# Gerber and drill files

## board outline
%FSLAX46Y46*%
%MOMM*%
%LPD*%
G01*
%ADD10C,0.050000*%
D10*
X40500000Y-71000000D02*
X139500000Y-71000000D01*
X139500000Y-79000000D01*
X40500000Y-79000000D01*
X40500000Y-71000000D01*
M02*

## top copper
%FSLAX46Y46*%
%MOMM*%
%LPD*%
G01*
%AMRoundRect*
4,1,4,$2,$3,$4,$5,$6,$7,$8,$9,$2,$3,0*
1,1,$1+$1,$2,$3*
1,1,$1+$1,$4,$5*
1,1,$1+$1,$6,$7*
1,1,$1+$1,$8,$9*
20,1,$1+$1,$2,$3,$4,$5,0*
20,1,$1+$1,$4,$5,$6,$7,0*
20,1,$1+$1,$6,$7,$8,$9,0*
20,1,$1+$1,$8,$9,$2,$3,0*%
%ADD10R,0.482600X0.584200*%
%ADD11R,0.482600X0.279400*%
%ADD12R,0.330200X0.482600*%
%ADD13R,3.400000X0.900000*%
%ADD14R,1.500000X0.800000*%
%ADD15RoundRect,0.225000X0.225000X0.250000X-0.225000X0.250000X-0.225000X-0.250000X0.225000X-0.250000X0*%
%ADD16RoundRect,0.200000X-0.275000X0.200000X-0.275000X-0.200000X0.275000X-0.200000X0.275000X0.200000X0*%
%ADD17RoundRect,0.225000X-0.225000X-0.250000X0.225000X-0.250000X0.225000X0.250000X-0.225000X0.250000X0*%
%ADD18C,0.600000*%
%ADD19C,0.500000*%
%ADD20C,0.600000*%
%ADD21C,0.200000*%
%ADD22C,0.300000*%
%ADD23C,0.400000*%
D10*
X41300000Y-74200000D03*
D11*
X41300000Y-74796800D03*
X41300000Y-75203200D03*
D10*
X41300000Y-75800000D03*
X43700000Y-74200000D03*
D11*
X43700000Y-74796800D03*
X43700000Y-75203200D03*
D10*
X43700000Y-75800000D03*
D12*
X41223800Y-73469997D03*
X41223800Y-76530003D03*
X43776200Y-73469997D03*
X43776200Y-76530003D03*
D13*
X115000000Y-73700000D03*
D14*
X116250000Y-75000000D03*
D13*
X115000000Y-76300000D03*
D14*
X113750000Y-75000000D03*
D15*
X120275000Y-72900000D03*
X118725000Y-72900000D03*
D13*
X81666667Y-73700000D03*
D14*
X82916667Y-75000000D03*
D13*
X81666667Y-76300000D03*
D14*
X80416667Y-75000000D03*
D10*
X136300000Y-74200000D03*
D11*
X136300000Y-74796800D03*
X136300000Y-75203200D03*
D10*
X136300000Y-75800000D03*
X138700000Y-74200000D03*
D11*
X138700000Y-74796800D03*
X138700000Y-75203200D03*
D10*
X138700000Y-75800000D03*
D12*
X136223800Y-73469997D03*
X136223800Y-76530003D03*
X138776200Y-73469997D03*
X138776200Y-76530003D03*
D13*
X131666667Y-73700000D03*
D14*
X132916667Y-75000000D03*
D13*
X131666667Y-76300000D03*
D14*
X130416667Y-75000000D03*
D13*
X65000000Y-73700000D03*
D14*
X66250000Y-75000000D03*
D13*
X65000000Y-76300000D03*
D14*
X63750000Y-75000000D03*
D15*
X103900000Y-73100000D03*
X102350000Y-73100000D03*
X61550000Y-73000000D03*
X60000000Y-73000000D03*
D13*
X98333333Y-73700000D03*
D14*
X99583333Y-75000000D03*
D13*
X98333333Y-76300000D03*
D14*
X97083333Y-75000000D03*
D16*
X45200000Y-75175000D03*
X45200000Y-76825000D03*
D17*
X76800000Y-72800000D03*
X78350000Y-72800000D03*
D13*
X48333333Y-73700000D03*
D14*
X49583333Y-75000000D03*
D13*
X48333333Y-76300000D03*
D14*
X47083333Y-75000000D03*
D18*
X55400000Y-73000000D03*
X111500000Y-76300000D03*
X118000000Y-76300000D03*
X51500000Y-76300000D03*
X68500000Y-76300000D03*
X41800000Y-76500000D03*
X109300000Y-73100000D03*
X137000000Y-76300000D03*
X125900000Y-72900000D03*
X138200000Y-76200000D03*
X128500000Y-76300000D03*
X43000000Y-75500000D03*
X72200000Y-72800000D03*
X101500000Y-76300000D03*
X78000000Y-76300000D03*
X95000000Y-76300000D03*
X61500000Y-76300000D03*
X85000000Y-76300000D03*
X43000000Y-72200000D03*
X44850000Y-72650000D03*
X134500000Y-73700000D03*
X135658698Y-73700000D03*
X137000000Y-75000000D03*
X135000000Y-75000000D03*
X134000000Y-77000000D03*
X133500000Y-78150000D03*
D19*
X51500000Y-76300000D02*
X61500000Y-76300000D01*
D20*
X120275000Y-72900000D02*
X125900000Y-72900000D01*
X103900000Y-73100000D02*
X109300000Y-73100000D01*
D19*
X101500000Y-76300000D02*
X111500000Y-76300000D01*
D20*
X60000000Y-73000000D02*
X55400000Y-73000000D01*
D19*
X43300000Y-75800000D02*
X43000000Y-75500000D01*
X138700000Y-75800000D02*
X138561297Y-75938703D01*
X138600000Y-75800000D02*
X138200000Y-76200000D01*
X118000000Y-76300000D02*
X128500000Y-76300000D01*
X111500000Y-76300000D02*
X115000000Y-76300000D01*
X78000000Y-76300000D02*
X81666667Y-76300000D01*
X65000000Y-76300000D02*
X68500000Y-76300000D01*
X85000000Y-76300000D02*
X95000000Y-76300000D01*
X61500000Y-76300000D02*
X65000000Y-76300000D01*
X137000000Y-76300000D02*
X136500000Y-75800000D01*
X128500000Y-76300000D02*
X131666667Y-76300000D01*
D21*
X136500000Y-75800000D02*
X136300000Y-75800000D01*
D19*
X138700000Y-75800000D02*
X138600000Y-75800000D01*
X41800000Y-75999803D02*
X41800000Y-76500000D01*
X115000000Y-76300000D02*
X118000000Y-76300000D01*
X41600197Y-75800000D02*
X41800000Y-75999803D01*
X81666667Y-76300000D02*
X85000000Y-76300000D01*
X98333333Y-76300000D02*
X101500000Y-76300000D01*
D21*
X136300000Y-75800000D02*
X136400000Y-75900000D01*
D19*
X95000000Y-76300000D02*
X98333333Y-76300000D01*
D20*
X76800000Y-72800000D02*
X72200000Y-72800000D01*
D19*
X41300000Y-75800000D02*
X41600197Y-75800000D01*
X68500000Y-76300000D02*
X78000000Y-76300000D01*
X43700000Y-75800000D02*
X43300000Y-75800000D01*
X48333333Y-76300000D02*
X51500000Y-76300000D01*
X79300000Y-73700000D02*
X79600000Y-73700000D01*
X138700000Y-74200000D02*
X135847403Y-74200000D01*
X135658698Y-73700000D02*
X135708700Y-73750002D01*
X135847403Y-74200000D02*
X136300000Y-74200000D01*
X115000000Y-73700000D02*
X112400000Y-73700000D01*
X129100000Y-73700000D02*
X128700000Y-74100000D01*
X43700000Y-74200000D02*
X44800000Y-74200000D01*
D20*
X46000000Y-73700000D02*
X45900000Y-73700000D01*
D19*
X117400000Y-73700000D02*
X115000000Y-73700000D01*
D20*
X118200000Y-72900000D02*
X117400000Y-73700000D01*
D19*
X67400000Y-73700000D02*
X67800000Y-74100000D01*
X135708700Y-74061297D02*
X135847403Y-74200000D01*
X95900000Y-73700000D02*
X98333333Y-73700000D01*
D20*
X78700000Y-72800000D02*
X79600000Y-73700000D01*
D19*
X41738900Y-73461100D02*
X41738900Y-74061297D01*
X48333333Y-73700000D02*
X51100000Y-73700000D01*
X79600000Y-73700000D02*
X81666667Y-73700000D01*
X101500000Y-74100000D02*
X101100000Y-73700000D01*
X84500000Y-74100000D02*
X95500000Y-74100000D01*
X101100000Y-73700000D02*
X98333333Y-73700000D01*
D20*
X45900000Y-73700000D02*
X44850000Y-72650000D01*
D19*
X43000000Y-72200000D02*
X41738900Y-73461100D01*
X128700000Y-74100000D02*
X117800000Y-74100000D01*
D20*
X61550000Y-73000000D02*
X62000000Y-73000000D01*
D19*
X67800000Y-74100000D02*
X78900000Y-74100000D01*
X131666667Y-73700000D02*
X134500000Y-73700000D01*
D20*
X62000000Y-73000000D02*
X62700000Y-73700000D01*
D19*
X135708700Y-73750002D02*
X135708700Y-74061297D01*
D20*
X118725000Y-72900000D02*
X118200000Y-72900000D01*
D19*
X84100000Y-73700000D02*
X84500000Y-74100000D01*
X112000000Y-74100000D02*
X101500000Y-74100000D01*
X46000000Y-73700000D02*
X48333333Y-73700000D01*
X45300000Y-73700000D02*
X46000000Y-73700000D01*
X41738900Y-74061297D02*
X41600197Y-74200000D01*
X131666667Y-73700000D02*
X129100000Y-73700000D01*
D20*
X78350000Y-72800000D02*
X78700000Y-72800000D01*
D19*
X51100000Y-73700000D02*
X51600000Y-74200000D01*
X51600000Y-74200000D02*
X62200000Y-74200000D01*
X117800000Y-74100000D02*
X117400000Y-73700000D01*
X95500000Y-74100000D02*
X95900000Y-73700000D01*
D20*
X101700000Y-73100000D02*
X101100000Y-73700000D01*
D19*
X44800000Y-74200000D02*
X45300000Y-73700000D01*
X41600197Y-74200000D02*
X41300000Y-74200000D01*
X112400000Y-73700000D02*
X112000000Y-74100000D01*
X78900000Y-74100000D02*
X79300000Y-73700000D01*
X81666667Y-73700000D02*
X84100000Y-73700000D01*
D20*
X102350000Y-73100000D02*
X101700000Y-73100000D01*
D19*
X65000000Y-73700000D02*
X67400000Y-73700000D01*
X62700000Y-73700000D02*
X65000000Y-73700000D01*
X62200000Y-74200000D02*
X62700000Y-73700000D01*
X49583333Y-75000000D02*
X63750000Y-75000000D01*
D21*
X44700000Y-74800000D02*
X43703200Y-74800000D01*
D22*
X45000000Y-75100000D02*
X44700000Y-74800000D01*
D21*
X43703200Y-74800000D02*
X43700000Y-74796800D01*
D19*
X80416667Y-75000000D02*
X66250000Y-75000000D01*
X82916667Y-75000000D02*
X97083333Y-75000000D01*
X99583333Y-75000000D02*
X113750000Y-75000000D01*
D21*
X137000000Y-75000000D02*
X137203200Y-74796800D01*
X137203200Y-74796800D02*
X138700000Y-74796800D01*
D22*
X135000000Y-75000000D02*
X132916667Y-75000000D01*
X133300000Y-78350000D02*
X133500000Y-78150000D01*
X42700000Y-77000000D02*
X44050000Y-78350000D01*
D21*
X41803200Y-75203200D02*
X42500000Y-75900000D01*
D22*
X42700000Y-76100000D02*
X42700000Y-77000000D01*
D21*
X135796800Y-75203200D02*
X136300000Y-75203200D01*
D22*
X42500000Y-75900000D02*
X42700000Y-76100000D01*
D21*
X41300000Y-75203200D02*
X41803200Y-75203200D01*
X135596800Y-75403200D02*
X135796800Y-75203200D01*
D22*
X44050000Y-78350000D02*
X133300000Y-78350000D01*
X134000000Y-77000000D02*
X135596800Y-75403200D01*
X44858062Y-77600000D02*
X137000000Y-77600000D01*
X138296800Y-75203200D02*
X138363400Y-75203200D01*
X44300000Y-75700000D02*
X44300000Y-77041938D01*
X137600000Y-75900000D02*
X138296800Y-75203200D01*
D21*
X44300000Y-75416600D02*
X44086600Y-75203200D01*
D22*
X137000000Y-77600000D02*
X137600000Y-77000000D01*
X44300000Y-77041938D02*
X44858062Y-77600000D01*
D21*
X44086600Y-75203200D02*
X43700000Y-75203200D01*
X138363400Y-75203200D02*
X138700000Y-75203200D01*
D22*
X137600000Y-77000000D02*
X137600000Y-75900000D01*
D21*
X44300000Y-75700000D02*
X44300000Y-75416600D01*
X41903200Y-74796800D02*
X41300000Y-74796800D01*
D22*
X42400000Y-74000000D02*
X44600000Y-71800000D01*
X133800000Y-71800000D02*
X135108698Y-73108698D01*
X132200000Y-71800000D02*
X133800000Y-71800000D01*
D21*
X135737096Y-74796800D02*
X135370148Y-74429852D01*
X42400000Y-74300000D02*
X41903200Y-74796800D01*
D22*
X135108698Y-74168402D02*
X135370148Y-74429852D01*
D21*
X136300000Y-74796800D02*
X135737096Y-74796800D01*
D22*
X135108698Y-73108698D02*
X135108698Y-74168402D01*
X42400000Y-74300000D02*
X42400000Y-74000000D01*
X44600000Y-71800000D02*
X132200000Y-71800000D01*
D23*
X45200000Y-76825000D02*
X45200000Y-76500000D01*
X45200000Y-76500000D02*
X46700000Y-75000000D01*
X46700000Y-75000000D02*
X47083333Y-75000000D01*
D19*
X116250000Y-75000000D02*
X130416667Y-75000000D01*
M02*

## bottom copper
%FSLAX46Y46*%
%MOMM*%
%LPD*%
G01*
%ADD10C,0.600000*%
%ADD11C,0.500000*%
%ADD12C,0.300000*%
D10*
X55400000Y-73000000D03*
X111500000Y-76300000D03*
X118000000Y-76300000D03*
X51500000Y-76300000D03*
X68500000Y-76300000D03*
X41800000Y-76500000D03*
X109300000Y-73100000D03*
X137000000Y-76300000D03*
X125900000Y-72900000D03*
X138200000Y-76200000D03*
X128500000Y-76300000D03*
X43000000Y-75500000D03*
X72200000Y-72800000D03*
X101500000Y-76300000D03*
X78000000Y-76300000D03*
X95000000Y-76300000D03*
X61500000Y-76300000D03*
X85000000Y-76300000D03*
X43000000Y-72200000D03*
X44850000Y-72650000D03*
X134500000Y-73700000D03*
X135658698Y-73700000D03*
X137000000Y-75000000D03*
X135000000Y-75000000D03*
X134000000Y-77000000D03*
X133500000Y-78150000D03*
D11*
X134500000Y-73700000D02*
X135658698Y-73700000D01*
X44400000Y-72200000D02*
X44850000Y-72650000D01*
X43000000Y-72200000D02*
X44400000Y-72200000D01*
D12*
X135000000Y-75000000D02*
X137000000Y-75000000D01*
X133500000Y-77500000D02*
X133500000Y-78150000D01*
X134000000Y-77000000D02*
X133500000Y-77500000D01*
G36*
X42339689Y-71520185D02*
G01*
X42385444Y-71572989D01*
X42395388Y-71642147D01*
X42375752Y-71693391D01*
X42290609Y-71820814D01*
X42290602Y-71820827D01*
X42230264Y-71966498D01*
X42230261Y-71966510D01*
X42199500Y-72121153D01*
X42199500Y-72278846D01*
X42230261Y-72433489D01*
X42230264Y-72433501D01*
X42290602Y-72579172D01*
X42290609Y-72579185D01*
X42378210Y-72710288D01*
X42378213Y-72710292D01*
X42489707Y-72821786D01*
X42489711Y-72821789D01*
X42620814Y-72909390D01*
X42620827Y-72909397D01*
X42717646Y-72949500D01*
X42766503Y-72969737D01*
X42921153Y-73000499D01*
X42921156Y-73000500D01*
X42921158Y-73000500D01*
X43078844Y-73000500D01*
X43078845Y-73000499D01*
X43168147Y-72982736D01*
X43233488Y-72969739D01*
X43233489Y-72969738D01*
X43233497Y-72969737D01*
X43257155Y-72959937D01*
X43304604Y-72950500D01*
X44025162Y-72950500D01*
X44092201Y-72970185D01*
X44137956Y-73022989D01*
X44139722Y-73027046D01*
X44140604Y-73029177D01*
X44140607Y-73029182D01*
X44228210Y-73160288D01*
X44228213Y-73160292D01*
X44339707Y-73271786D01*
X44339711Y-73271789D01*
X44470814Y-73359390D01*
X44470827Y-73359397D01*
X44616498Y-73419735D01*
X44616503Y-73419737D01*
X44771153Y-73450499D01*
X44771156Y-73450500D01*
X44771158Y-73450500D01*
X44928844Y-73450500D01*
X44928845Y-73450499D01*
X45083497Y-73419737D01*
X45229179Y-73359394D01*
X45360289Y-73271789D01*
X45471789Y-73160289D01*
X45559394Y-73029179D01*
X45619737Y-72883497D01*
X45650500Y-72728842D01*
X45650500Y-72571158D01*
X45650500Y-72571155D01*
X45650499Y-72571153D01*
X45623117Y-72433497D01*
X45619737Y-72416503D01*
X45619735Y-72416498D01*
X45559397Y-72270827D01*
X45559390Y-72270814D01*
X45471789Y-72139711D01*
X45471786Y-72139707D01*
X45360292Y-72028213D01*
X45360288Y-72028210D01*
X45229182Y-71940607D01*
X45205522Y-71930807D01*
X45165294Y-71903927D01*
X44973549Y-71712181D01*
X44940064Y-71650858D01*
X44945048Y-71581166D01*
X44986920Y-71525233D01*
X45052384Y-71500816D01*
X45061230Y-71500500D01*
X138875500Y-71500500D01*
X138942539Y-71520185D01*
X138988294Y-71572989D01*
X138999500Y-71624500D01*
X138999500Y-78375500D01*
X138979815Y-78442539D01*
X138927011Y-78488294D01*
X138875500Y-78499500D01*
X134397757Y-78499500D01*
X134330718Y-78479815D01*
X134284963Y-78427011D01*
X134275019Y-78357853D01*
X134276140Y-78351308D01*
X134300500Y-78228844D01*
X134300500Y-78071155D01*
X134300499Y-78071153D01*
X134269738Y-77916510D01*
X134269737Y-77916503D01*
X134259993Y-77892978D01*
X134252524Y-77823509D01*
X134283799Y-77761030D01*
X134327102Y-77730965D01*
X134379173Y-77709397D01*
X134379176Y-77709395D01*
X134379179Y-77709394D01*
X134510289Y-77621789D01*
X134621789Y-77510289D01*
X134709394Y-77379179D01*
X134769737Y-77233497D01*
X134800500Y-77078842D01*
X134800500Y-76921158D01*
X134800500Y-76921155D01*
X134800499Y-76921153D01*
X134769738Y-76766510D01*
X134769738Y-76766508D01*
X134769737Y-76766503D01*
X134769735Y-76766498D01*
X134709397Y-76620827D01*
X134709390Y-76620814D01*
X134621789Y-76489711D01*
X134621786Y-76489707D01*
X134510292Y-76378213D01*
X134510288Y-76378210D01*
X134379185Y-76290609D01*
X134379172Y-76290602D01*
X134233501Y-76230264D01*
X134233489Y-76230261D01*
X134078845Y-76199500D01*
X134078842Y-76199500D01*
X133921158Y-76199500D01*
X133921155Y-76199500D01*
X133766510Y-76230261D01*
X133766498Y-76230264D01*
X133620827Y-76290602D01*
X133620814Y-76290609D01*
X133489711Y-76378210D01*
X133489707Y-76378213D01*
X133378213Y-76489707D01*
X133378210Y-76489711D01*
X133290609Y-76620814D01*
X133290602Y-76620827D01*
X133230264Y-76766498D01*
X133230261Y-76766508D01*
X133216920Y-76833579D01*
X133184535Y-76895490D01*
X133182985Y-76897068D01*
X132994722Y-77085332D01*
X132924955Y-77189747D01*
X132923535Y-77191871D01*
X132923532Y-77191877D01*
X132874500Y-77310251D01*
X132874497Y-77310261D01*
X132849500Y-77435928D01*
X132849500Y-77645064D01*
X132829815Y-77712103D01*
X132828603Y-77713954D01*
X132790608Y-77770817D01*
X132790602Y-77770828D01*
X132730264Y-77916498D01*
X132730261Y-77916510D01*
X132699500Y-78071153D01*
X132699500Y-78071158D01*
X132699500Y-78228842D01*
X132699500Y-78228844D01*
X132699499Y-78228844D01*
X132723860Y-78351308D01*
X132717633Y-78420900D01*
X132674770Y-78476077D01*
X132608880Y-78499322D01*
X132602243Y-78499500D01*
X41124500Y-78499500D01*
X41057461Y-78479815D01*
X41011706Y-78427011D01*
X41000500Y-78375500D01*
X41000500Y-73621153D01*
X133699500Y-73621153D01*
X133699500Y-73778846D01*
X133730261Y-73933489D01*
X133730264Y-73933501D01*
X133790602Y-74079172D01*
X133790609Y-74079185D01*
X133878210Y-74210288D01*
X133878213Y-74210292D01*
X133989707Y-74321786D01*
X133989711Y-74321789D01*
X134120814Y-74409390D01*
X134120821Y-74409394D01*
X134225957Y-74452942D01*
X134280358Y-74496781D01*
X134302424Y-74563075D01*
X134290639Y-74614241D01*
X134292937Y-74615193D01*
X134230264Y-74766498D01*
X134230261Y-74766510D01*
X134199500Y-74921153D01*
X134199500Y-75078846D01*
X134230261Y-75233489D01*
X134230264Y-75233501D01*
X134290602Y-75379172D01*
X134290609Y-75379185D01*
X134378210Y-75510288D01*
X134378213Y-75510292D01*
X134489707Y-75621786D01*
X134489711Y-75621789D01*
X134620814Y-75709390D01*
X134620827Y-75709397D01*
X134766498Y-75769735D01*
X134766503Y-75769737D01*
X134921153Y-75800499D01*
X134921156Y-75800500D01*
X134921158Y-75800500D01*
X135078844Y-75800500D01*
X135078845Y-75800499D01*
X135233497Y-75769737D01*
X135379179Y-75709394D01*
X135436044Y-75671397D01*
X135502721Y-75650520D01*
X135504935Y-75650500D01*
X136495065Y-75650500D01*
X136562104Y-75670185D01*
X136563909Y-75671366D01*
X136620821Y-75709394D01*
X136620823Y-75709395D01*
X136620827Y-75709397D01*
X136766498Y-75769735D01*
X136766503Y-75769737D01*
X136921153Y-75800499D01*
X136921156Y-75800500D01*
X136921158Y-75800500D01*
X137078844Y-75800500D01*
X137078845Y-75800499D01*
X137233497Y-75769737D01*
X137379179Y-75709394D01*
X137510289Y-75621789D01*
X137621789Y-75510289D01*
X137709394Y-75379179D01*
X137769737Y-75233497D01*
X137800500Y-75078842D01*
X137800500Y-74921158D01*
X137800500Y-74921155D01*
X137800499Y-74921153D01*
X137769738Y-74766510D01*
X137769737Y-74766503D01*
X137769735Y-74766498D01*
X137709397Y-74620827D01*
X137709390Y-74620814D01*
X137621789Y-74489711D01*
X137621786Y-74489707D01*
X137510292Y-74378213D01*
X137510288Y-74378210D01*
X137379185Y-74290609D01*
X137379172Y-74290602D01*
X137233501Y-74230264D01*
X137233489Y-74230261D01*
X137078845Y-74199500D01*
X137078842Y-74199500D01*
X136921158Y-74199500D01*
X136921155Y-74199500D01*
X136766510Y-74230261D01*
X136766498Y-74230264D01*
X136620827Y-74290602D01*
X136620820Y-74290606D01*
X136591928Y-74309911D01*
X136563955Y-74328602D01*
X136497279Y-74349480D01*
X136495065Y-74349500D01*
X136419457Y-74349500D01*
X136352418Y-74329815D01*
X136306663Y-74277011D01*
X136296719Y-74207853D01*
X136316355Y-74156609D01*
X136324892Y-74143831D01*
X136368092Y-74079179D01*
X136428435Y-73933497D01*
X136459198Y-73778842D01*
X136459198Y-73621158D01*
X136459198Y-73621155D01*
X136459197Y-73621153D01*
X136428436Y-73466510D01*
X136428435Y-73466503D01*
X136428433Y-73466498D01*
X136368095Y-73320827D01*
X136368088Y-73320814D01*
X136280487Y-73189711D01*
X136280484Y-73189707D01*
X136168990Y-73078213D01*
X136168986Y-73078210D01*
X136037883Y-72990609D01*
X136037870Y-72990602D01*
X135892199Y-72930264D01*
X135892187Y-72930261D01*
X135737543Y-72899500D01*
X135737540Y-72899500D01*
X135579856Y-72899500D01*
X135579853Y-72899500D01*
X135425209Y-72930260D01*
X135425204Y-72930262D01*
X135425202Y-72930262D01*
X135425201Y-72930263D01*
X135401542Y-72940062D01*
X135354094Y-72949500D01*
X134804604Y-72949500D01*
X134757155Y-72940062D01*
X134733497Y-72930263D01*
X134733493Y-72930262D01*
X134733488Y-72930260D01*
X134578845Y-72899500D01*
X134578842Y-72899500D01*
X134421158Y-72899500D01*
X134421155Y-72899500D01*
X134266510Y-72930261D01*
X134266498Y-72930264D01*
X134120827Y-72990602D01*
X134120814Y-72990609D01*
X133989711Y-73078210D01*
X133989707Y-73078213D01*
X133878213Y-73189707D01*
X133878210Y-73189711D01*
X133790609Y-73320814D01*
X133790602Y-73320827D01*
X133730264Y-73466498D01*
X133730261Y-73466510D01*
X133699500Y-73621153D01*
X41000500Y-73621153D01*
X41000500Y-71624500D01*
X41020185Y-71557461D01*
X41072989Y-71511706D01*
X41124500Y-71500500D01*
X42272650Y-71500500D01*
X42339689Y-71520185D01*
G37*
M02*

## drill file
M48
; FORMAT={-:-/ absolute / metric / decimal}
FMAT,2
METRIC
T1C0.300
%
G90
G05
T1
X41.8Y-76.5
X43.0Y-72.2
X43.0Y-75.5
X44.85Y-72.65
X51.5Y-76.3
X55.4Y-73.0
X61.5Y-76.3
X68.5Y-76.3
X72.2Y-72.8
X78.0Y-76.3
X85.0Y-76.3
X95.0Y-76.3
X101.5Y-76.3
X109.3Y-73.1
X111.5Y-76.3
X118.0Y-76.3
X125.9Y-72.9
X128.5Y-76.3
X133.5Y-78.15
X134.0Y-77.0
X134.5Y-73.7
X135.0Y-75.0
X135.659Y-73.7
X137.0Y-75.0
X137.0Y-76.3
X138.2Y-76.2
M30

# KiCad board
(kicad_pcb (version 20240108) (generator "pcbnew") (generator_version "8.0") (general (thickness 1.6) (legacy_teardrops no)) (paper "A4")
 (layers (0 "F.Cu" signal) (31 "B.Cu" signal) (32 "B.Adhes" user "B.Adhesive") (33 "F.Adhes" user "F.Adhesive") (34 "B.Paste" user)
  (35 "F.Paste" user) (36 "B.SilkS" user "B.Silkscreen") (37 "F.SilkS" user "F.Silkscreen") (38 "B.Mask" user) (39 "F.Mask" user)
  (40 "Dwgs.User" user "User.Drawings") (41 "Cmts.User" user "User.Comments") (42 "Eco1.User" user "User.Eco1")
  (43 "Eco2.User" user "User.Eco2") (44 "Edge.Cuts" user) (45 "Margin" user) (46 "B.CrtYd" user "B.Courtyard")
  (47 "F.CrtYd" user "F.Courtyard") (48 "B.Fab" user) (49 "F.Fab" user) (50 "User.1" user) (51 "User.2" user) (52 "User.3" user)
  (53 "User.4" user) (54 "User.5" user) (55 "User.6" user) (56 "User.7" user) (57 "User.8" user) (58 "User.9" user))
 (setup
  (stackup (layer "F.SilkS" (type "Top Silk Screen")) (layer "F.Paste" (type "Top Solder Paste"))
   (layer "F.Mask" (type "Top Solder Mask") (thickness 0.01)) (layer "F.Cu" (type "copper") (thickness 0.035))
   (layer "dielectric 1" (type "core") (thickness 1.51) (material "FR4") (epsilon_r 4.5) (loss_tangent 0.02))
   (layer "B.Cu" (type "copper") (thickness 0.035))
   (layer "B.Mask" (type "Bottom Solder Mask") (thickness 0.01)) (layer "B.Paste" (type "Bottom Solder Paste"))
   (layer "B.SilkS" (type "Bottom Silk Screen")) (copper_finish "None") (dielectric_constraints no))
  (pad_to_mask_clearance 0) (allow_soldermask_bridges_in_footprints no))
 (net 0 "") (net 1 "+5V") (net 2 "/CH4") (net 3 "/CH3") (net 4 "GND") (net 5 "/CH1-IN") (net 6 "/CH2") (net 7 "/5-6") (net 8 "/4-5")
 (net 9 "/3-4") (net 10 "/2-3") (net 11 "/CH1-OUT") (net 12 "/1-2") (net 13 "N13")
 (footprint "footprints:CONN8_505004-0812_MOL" (layer "F.Cu") (at 42.5 75 90)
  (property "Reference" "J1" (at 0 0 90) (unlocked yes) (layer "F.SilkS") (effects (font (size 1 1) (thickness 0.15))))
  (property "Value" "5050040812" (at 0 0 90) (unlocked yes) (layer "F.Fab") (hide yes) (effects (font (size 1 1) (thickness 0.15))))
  (pad "1" smd rect (at 0.8 -1.2 90) (size 0.5842 0.4826) (layers "F.Cu" "F.Paste" "F.Mask") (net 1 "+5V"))
  (pad "2" smd rect (at 0.2032 -1.2 90) (size 0.2794 0.4826) (layers "F.Cu" "F.Paste" "F.Mask") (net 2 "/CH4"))
  (pad "3" smd rect (at -0.2032 -1.2 90) (size 0.2794 0.4826) (layers "F.Cu" "F.Paste" "F.Mask") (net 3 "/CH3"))
  (pad "4" smd rect (at -0.8 -1.2 90) (size 0.5842 0.4826) (layers "F.Cu" "F.Paste" "F.Mask") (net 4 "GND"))
  (pad "5" smd rect (at 0.8 1.2 90) (size 0.5842 0.4826) (layers "F.Cu" "F.Paste" "F.Mask") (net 1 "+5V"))
  (pad "6" smd rect (at 0.2032 1.2 90) (size 0.2794 0.4826) (layers "F.Cu" "F.Paste" "F.Mask") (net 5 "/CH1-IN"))
  (pad "7" smd rect (at -0.2032 1.2 90) (size 0.2794 0.4826) (layers "F.Cu" "F.Paste" "F.Mask") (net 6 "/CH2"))
  (pad "8" smd rect (at -0.8 1.2 90) (size 0.5842 0.4826) (layers "F.Cu" "F.Paste" "F.Mask") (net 4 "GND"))
  (pad "9" smd rect (at 1.530003 -1.2762 90) (size 0.4826 0.3302) (layers "F.Cu" "F.Paste" "F.Mask"))
  (pad "10" smd rect (at -1.530003 -1.2762 90) (size 0.4826 0.3302) (layers "F.Cu" "F.Paste" "F.Mask"))
  (pad "11" smd rect (at 1.530003 1.2762 90) (size 0.4826 0.3302) (layers "F.Cu" "F.Paste" "F.Mask"))
  (pad "12" smd rect (at -1.530003 1.2762 90) (size 0.4826 0.3302) (layers "F.Cu" "F.Paste" "F.Mask")))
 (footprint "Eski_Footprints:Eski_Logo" (layer "F.Cu") (at 90 76.9)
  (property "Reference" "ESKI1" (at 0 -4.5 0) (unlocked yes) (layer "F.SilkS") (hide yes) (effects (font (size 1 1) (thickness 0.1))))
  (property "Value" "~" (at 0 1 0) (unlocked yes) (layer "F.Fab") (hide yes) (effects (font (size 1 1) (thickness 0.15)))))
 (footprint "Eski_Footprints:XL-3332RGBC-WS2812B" (layer "F.Cu") (at 115 75)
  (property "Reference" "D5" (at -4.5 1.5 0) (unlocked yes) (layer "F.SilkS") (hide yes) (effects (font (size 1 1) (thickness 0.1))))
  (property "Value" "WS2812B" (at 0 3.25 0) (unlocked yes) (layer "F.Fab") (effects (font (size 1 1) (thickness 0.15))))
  (pad "1" smd rect (at 0 -1.3) (size 3.4 0.9) (layers "F.Cu" "F.Paste" "F.Mask") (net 1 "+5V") (thermal_bridge_angle 45))
  (pad "2" smd rect (at 1.25 0) (size 1.5 0.8) (layers "F.Cu" "F.Paste" "F.Mask") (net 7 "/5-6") (thermal_bridge_angle 45))
  (pad "3" smd rect (at 0 1.3) (size 3.4 0.9) (layers "F.Cu" "F.Paste" "F.Mask") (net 4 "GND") (thermal_bridge_angle 45))
  (pad "4" smd rect (at -1.25 0) (size 1.5 0.8) (layers "F.Cu" "F.Paste" "F.Mask") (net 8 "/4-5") (thermal_bridge_angle 45)))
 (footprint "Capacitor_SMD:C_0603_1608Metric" (layer "F.Cu") (at 119.5 72.9 180)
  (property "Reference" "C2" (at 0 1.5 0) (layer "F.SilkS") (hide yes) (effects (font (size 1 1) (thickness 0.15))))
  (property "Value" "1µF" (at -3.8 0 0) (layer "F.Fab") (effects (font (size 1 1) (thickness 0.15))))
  (pad "1" smd roundrect (at -0.775 0 180) (size 0.9 0.95) (layers "F.Cu" "F.Paste" "F.Mask") (roundrect_rratio 0.25) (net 4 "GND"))
  (pad "2" smd roundrect (at 0.775 0 180) (size 0.9 0.95) (layers "F.Cu" "F.Paste" "F.Mask") (roundrect_rratio 0.25) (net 1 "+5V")))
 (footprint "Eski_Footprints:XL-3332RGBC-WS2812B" (layer "F.Cu") (at 81.666667 75)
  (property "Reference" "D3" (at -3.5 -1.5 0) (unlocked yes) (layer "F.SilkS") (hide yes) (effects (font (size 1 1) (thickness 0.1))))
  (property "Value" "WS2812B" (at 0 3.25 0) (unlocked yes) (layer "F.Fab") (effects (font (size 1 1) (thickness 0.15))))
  (pad "1" smd rect (at 0 -1.3) (size 3.4 0.9) (layers "F.Cu" "F.Paste" "F.Mask") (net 1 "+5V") (thermal_bridge_angle 45))
  (pad "2" smd rect (at 1.25 0) (size 1.5 0.8) (layers "F.Cu" "F.Paste" "F.Mask") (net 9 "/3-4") (thermal_bridge_angle 45))
  (pad "3" smd rect (at 0 1.3) (size 3.4 0.9) (layers "F.Cu" "F.Paste" "F.Mask") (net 4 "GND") (thermal_bridge_angle 45))
  (pad "4" smd rect (at -1.25 0) (size 1.5 0.8) (layers "F.Cu" "F.Paste" "F.Mask") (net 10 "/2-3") (thermal_bridge_angle 45)))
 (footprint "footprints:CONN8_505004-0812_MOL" (layer "F.Cu") (at 137.5 75 90)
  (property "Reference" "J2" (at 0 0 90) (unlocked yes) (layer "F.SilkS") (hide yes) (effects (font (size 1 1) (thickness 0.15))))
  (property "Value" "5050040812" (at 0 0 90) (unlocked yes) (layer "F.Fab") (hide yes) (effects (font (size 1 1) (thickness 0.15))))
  (pad "1" smd rect (at 0.8 -1.2 90) (size 0.5842 0.4826) (layers "F.Cu" "F.Paste" "F.Mask") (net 1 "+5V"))
  (pad "2" smd rect (at 0.2032 -1.2 90) (size 0.2794 0.4826) (layers "F.Cu" "F.Paste" "F.Mask") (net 2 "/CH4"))
  (pad "3" smd rect (at -0.2032 -1.2 90) (size 0.2794 0.4826) (layers "F.Cu" "F.Paste" "F.Mask") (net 3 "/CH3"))
  (pad "4" smd rect (at -0.8 -1.2 90) (size 0.5842 0.4826) (layers "F.Cu" "F.Paste" "F.Mask") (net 4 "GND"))
  (pad "5" smd rect (at 0.8 1.2 90) (size 0.5842 0.4826) (layers "F.Cu" "F.Paste" "F.Mask") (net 1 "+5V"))
  (pad "6" smd rect (at 0.2032 1.2 90) (size 0.2794 0.4826) (layers "F.Cu" "F.Paste" "F.Mask") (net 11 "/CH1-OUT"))
  (pad "7" smd rect (at -0.2032 1.2 90) (size 0.2794 0.4826) (layers "F.Cu" "F.Paste" "F.Mask") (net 6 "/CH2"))
  (pad "8" smd rect (at -0.8 1.2 90) (size 0.5842 0.4826) (layers "F.Cu" "F.Paste" "F.Mask") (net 4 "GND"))
  (pad "9" smd rect (at 1.530003 -1.2762 90) (size 0.4826 0.3302) (layers "F.Cu" "F.Paste" "F.Mask"))
  (pad "10" smd rect (at -1.530003 -1.2762 90) (size 0.4826 0.3302) (layers "F.Cu" "F.Paste" "F.Mask"))
  (pad "11" smd rect (at 1.530003 1.2762 90) (size 0.4826 0.3302) (layers "F.Cu" "F.Paste" "F.Mask"))
  (pad "12" smd rect (at -1.530003 1.2762 90) (size 0.4826 0.3302) (layers "F.Cu" "F.Paste" "F.Mask")))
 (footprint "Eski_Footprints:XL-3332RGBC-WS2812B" (layer "F.Cu") (at 131.666667 75)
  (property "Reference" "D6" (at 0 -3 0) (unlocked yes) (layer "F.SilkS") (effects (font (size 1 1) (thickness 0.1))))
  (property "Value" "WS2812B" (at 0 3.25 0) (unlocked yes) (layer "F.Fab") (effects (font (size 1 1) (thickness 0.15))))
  (pad "1" smd rect (at 0 -1.3) (size 3.4 0.9) (layers "F.Cu" "F.Paste" "F.Mask") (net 1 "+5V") (thermal_bridge_angle 45))
  (pad "2" smd rect (at 1.25 0) (size 1.5 0.8) (layers "F.Cu" "F.Paste" "F.Mask") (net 11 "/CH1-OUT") (thermal_bridge_angle 45))
  (pad "3" smd rect (at 0 1.3) (size 3.4 0.9) (layers "F.Cu" "F.Paste" "F.Mask") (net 4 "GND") (thermal_bridge_angle 45))
  (pad "4" smd rect (at -1.25 0) (size 1.5 0.8) (layers "F.Cu" "F.Paste" "F.Mask") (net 7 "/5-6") (thermal_bridge_angle 45)))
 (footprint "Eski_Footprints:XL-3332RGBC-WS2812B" (layer "F.Cu") (at 65 75)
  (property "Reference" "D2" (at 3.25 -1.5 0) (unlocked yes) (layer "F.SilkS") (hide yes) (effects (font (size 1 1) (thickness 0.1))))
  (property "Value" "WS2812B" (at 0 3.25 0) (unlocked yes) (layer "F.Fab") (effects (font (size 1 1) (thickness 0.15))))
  (pad "1" smd rect (at 0 -1.3) (size 3.4 0.9) (layers "F.Cu" "F.Paste" "F.Mask") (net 1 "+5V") (thermal_bridge_angle 45))
  (pad "2" smd rect (at 1.25 0) (size 1.5 0.8) (layers "F.Cu" "F.Paste" "F.Mask") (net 10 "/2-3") (thermal_bridge_angle 45))
  (pad "3" smd rect (at 0 1.3) (size 3.4 0.9) (layers "F.Cu" "F.Paste" "F.Mask") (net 4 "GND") (thermal_bridge_angle 45))
  (pad "4" smd rect (at -1.25 0) (size 1.5 0.8) (layers "F.Cu" "F.Paste" "F.Mask") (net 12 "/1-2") (thermal_bridge_angle 45)))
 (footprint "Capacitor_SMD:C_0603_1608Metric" (layer "F.Cu") (at 103.125 73.1 180)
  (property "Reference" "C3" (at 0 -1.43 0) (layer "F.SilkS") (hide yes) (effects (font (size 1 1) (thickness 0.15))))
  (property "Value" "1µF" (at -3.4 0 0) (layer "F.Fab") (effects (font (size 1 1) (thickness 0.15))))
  (pad "1" smd roundrect (at -0.775 0 180) (size 0.9 0.95) (layers "F.Cu" "F.Paste" "F.Mask") (roundrect_rratio 0.25) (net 4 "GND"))
  (pad "2" smd roundrect (at 0.775 0 180) (size 0.9 0.95) (layers "F.Cu" "F.Paste" "F.Mask") (roundrect_rratio 0.25) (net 1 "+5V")))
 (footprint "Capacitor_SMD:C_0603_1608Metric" (layer "F.Cu") (at 60.775 73 180)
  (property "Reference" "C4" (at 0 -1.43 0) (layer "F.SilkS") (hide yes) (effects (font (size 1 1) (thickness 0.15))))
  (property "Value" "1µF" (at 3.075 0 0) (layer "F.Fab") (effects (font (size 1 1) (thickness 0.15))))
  (pad "1" smd roundrect (at -0.775 0 180) (size 0.9 0.95) (layers "F.Cu" "F.Paste" "F.Mask") (roundrect_rratio 0.25) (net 1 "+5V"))
  (pad "2" smd roundrect (at 0.775 0 180) (size 0.9 0.95) (layers "F.Cu" "F.Paste" "F.Mask") (roundrect_rratio 0.25) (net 4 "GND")))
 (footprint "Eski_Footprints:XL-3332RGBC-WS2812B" (layer "F.Cu") (at 98.333333 75)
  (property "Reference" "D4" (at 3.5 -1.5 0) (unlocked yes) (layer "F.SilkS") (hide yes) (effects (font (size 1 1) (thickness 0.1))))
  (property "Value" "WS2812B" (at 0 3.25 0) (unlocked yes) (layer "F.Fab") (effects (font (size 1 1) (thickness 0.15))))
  (pad "1" smd rect (at 0 -1.3) (size 3.4 0.9) (layers "F.Cu" "F.Paste" "F.Mask") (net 1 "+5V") (thermal_bridge_angle 45))
  (pad "2" smd rect (at 1.25 0) (size 1.5 0.8) (layers "F.Cu" "F.Paste" "F.Mask") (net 8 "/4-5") (thermal_bridge_angle 45))
  (pad "3" smd rect (at 0 1.3) (size 3.4 0.9) (layers "F.Cu" "F.Paste" "F.Mask") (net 4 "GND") (thermal_bridge_angle 45))
  (pad "4" smd rect (at -1.25 0) (size 1.5 0.8) (layers "F.Cu" "F.Paste" "F.Mask") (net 9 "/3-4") (thermal_bridge_angle 45)))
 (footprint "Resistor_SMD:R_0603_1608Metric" (layer "F.Cu") (at 45.2 76 -90)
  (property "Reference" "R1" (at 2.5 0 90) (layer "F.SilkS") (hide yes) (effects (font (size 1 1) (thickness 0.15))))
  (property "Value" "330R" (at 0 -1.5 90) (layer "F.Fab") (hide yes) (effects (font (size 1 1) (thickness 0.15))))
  (pad "1" smd roundrect (at -0.825 0 270) (size 0.8 0.95) (layers "F.Cu" "F.Paste" "F.Mask") (roundrect_rratio 0.25) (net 5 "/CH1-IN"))
  (pad "2" smd roundrect (at 0.825 0 270) (size 0.8 0.95) (layers "F.Cu" "F.Paste" "F.Mask") (roundrect_rratio 0.25) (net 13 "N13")))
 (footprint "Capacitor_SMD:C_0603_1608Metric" (layer "F.Cu") (at 77.575 72.8)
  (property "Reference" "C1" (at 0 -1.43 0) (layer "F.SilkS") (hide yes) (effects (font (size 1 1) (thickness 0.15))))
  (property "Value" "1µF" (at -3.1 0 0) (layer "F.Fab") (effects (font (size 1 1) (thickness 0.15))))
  (pad "1" smd roundrect (at -0.775 0) (size 0.9 0.95) (layers "F.Cu" "F.Paste" "F.Mask") (roundrect_rratio 0.25) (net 4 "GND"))
  (pad "2" smd roundrect (at 0.775 0) (size 0.9 0.95) (layers "F.Cu" "F.Paste" "F.Mask") (roundrect_rratio 0.25) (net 1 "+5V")))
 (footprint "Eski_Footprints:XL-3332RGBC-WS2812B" (layer "F.Cu") (at 48.333333 75)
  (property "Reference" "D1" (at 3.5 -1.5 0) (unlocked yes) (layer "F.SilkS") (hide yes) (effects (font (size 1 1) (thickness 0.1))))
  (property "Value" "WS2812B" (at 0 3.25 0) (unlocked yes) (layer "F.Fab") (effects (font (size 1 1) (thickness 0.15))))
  (pad "1" smd rect (at 0 -1.3) (size 3.4 0.9) (layers "F.Cu" "F.Paste" "F.Mask") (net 1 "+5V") (thermal_bridge_angle 45))
  (pad "2" smd rect (at 1.25 0) (size 1.5 0.8) (layers "F.Cu" "F.Paste" "F.Mask") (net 12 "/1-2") (thermal_bridge_angle 45))
  (pad "3" smd rect (at 0 1.3) (size 3.4 0.9) (layers "F.Cu" "F.Paste" "F.Mask") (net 4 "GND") (thermal_bridge_angle 45))
  (pad "4" smd rect (at -1.25 0) (size 1.5 0.8) (layers "F.Cu" "F.Paste" "F.Mask") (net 13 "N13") (thermal_bridge_angle 45)))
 (gr_rect (start 40.5 71) (end 139.5 79) (stroke (width 0.05) (type default)) (fill none) (layer "Edge.Cuts"))
 (segment (start 51.5 76.3) (end 61.5 76.3) (width 0.5) (layer "F.Cu") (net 4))
 (segment (start 120.275 72.9) (end 125.9 72.9) (width 0.6) (layer "F.Cu") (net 4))
 (segment (start 103.9 73.1) (end 109.3 73.1) (width 0.6) (layer "F.Cu") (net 4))
 (segment (start 101.5 76.3) (end 111.5 76.3) (width 0.5) (layer "F.Cu") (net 4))
 (segment (start 60 73) (end 55.4 73) (width 0.6) (layer "F.Cu") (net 4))
 (segment (start 43.3 75.8) (end 43 75.5) (width 0.5) (layer "F.Cu") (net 4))
 (segment (start 138.7 75.8) (end 138.561297 75.938703) (width 0.5) (layer "F.Cu") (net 4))
 (segment (start 138.6 75.8) (end 138.2 76.2) (width 0.5) (layer "F.Cu") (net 4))
 (segment (start 118 76.3) (end 128.5 76.3) (width 0.5) (layer "F.Cu") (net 4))
 (segment (start 111.5 76.3) (end 115 76.3) (width 0.5) (layer "F.Cu") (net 4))
 (segment (start 78 76.3) (end 81.666667 76.3) (width 0.5) (layer "F.Cu") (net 4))
 (segment (start 65 76.3) (end 68.5 76.3) (width 0.5) (layer "F.Cu") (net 4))
 (segment (start 85 76.3) (end 95 76.3) (width 0.5) (layer "F.Cu") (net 4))
 (segment (start 61.5 76.3) (end 65 76.3) (width 0.5) (layer "F.Cu") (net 4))
 (segment (start 137 76.3) (end 136.5 75.8) (width 0.5) (layer "F.Cu") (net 4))
 (segment (start 128.5 76.3) (end 131.666667 76.3) (width 0.5) (layer "F.Cu") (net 4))
 (segment (start 136.5 75.8) (end 136.3 75.8) (width 0.2) (layer "F.Cu") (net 4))
 (segment (start 138.7 75.8) (end 138.6 75.8) (width 0.5) (layer "F.Cu") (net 4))
 (segment (start 41.8 75.999803) (end 41.8 76.5) (width 0.5) (layer "F.Cu") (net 4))
 (segment (start 115 76.3) (end 118 76.3) (width 0.5) (layer "F.Cu") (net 4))
 (segment (start 41.600197 75.8) (end 41.8 75.999803) (width 0.5) (layer "F.Cu") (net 4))
 (segment (start 81.666667 76.3) (end 85 76.3) (width 0.5) (layer "F.Cu") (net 4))
 (segment (start 98.333333 76.3) (end 101.5 76.3) (width 0.5) (layer "F.Cu") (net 4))
 (segment (start 136.3 75.8) (end 136.4 75.9) (width 0.2) (layer "F.Cu") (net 4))
 (segment (start 95 76.3) (end 98.333333 76.3) (width 0.5) (layer "F.Cu") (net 4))
 (segment (start 76.8 72.8) (end 72.2 72.8) (width 0.6) (layer "F.Cu") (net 4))
 (segment (start 41.3 75.8) (end 41.600197 75.8) (width 0.5) (layer "F.Cu") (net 4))
 (segment (start 68.5 76.3) (end 78 76.3) (width 0.5) (layer "F.Cu") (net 4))
 (segment (start 43.7 75.8) (end 43.3 75.8) (width 0.5) (layer "F.Cu") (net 4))
 (segment (start 48.333333 76.3) (end 51.5 76.3) (width 0.5) (layer "F.Cu") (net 4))
 (via (at 55.4 73) (size 0.6) (drill 0.3) (layers "F.Cu" "B.Cu") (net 4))
 (via (at 111.5 76.3) (size 0.6) (drill 0.3) (layers "F.Cu" "B.Cu") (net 4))
 (via (at 118 76.3) (size 0.6) (drill 0.3) (layers "F.Cu" "B.Cu") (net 4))
 (via (at 51.5 76.3) (size 0.6) (drill 0.3) (layers "F.Cu" "B.Cu") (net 4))
 (via (at 68.5 76.3) (size 0.6) (drill 0.3) (layers "F.Cu" "B.Cu") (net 4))
 (via (at 41.8 76.5) (size 0.6) (drill 0.3) (layers "F.Cu" "B.Cu") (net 4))
 (via (at 109.3 73.1) (size 0.6) (drill 0.3) (layers "F.Cu" "B.Cu") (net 4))
 (via (at 137 76.3) (size 0.6) (drill 0.3) (layers "F.Cu" "B.Cu") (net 4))
 (via (at 125.9 72.9) (size 0.6) (drill 0.3) (layers "F.Cu" "B.Cu") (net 4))
 (via (at 138.2 76.2) (size 0.6) (drill 0.3) (layers "F.Cu" "B.Cu") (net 4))
 (via (at 128.5 76.3) (size 0.6) (drill 0.3) (layers "F.Cu" "B.Cu") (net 4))
 (via (at 43 75.5) (size 0.6) (drill 0.3) (layers "F.Cu" "B.Cu") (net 4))
 (via (at 72.2 72.8) (size 0.6) (drill 0.3) (layers "F.Cu" "B.Cu") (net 4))
 (via (at 101.5 76.3) (size 0.6) (drill 0.3) (layers "F.Cu" "B.Cu") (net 4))
 (via (at 78 76.3) (size 0.6) (drill 0.3) (layers "F.Cu" "B.Cu") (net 4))
 (via (at 95 76.3) (size 0.6) (drill 0.3) (layers "F.Cu" "B.Cu") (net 4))
 (via (at 61.5 76.3) (size 0.6) (drill 0.3) (layers "F.Cu" "B.Cu") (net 4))
 (via (at 85 76.3) (size 0.6) (drill 0.3) (layers "F.Cu" "B.Cu") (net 4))
 (segment (start 79.3 73.7) (end 79.6 73.7) (width 0.5) (layer "F.Cu") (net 1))
 (segment (start 138.7 74.2) (end 135.847403 74.2) (width 0.5) (layer "F.Cu") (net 1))
 (segment (start 135.658698 73.7) (end 135.7087 73.750002) (width 0.5) (layer "F.Cu") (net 1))
 (segment (start 135.847403 74.2) (end 136.3 74.2) (width 0.5) (layer "F.Cu") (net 1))
 (segment (start 115 73.7) (end 112.4 73.7) (width 0.5) (layer "F.Cu") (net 1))
 (segment (start 129.1 73.7) (end 128.7 74.1) (width 0.5) (layer "F.Cu") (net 1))
 (segment (start 43.7 74.2) (end 44.8 74.2) (width 0.5) (layer "F.Cu") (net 1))
 (segment (start 46 73.7) (end 45.9 73.7) (width 0.6) (layer "F.Cu") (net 1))
 (segment (start 117.4 73.7) (end 115 73.7) (width 0.5) (layer "F.Cu") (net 1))
 (segment (start 118.2 72.9) (end 117.4 73.7) (width 0.6) (layer "F.Cu") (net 1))
 (segment (start 67.4 73.7) (end 67.8 74.1) (width 0.5) (layer "F.Cu") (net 1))
 (segment (start 135.7087 74.061297) (end 135.847403 74.2) (width 0.5) (layer "F.Cu") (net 1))
 (segment (start 95.9 73.7) (end 98.333333 73.7) (width 0.5) (layer "F.Cu") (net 1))
 (segment (start 78.7 72.8) (end 79.6 73.7) (width 0.6) (layer "F.Cu") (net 1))
 (segment (start 41.7389 73.4611) (end 41.7389 74.061297) (width 0.5) (layer "F.Cu") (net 1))
 (segment (start 48.333333 73.7) (end 51.1 73.7) (width 0.5) (layer "F.Cu") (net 1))
 (segment (start 79.6 73.7) (end 81.666667 73.7) (width 0.5) (layer "F.Cu") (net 1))
 (segment (start 101.5 74.1) (end 101.1 73.7) (width 0.5) (layer "F.Cu") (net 1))
 (segment (start 84.5 74.1) (end 95.5 74.1) (width 0.5) (layer "F.Cu") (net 1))
 (segment (start 101.1 73.7) (end 98.333333 73.7) (width 0.5) (layer "F.Cu") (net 1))
 (segment (start 45.9 73.7) (end 44.85 72.65) (width 0.6) (layer "F.Cu") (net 1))
 (segment (start 43 72.2) (end 41.7389 73.4611) (width 0.5) (layer "F.Cu") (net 1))
 (segment (start 128.7 74.1) (end 117.8 74.1) (width 0.5) (layer "F.Cu") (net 1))
 (segment (start 61.55 73) (end 62 73) (width 0.6) (layer "F.Cu") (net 1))
 (segment (start 67.8 74.1) (end 78.9 74.1) (width 0.5) (layer "F.Cu") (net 1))
 (segment (start 131.666667 73.7) (end 134.5 73.7) (width 0.5) (layer "F.Cu") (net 1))
 (segment (start 62 73) (end 62.7 73.7) (width 0.6) (layer "F.Cu") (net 1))
 (segment (start 135.7087 73.750002) (end 135.7087 74.061297) (width 0.5) (layer "F.Cu") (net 1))
 (segment (start 118.725 72.9) (end 118.2 72.9) (width 0.6) (layer "F.Cu") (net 1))
 (segment (start 84.1 73.7) (end 84.5 74.1) (width 0.5) (layer "F.Cu") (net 1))
 (segment (start 112 74.1) (end 101.5 74.1) (width 0.5) (layer "F.Cu") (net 1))
 (segment (start 46 73.7) (end 48.333333 73.7) (width 0.5) (layer "F.Cu") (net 1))
 (segment (start 45.3 73.7) (end 46 73.7) (width 0.5) (layer "F.Cu") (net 1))
 (segment (start 41.7389 74.061297) (end 41.600197 74.2) (width 0.5) (layer "F.Cu") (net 1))
 (segment (start 131.666667 73.7) (end 129.1 73.7) (width 0.5) (layer "F.Cu") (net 1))
 (segment (start 78.35 72.8) (end 78.7 72.8) (width 0.6) (layer "F.Cu") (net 1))
 (segment (start 51.1 73.7) (end 51.6 74.2) (width 0.5) (layer "F.Cu") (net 1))
 (segment (start 51.6 74.2) (end 62.2 74.2) (width 0.5) (layer "F.Cu") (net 1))
 (segment (start 117.8 74.1) (end 117.4 73.7) (width 0.5) (layer "F.Cu") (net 1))
 (segment (start 95.5 74.1) (end 95.9 73.7) (width 0.5) (layer "F.Cu") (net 1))
 (segment (start 101.7 73.1) (end 101.1 73.7) (width 0.6) (layer "F.Cu") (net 1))
 (segment (start 44.8 74.2) (end 45.3 73.7) (width 0.5) (layer "F.Cu") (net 1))
 (segment (start 41.600197 74.2) (end 41.3 74.2) (width 0.5) (layer "F.Cu") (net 1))
 (segment (start 112.4 73.7) (end 112 74.1) (width 0.5) (layer "F.Cu") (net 1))
 (segment (start 78.9 74.1) (end 79.3 73.7) (width 0.5) (layer "F.Cu") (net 1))
 (segment (start 81.666667 73.7) (end 84.1 73.7) (width 0.5) (layer "F.Cu") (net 1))
 (segment (start 102.35 73.1) (end 101.7 73.1) (width 0.6) (layer "F.Cu") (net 1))
 (segment (start 65 73.7) (end 67.4 73.7) (width 0.5) (layer "F.Cu") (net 1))
 (segment (start 62.7 73.7) (end 65 73.7) (width 0.5) (layer "F.Cu") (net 1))
 (segment (start 62.2 74.2) (end 62.7 73.7) (width 0.5) (layer "F.Cu") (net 1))
 (via (at 43 72.2) (size 0.6) (drill 0.3) (layers "F.Cu" "B.Cu") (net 1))
 (via (at 44.85 72.65) (size 0.6) (drill 0.3) (layers "F.Cu" "B.Cu") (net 1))
 (via (at 134.5 73.7) (size 0.6) (drill 0.3) (layers "F.Cu" "B.Cu") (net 1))
 (via (at 135.658698 73.7) (size 0.6) (drill 0.3) (layers "F.Cu" "B.Cu") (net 1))
 (segment (start 134.5 73.7) (end 135.658698 73.7) (width 0.5) (layer "B.Cu") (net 1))
 (segment (start 44.4 72.2) (end 44.85 72.65) (width 0.5) (layer "B.Cu") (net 1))
 (segment (start 43 72.2) (end 44.4 72.2) (width 0.5) (layer "B.Cu") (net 1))
 (segment (start 49.583333 75) (end 63.75 75) (width 0.5) (layer "F.Cu") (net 12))
 (segment (start 44.7 74.8) (end 43.7032 74.8) (width 0.2) (layer "F.Cu") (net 5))
 (segment (start 45 75.1) (end 44.7 74.8) (width 0.3) (layer "F.Cu") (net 5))
 (segment (start 43.7032 74.8) (end 43.7 74.7968) (width 0.2) (layer "F.Cu") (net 5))
 (segment (start 80.416667 75) (end 66.25 75) (width 0.5) (layer "F.Cu") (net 10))
 (segment (start 82.916667 75) (end 97.083333 75) (width 0.5) (layer "F.Cu") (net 9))
 (segment (start 99.583333 75) (end 113.75 75) (width 0.5) (layer "F.Cu") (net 8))
 (segment (start 137 75) (end 137.2032 74.7968) (width 0.2) (layer "F.Cu") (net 11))
 (segment (start 137.2032 74.7968) (end 138.7 74.7968) (width 0.2) (layer "F.Cu") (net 11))
 (segment (start 135 75) (end 132.916667 75) (width 0.3) (layer "F.Cu") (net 11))
 (via (at 137 75) (size 0.6) (drill 0.3) (layers "F.Cu" "B.Cu") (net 11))
 (via (at 135 75) (size 0.6) (drill 0.3) (layers "F.Cu" "B.Cu") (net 11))
 (segment (start 135 75) (end 137 75) (width 0.3) (layer "B.Cu") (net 11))
 (segment (start 133.3 78.35) (end 133.5 78.15) (width 0.3) (layer "F.Cu") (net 3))
 (segment (start 42.7 77) (end 44.05 78.35) (width 0.3) (layer "F.Cu") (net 3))
 (segment (start 41.8032 75.2032) (end 42.5 75.9) (width 0.2) (layer "F.Cu") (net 3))
 (segment (start 42.7 76.1) (end 42.7 77) (width 0.3) (layer "F.Cu") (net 3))
 (segment (start 135.7968 75.2032) (end 136.3 75.2032) (width 0.2) (layer "F.Cu") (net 3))
 (segment (start 42.5 75.9) (end 42.7 76.1) (width 0.3) (layer "F.Cu") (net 3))
 (segment (start 41.3 75.2032) (end 41.8032 75.2032) (width 0.2) (layer "F.Cu") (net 3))
 (segment (start 135.5968 75.4032) (end 135.7968 75.2032) (width 0.2) (layer "F.Cu") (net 3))
 (segment (start 44.05 78.35) (end 133.3 78.35) (width 0.3) (layer "F.Cu") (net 3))
 (segment (start 134 77) (end 135.5968 75.4032) (width 0.3) (layer "F.Cu") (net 3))
 (via (at 134 77) (size 0.6) (drill 0.3) (layers "F.Cu" "B.Cu") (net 3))
 (via (at 133.5 78.15) (size 0.6) (drill 0.3) (layers "F.Cu" "B.Cu") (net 3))
 (segment (start 133.5 77.5) (end 133.5 78.15) (width 0.3) (layer "B.Cu") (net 3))
 (segment (start 134 77) (end 133.5 77.5) (width 0.3) (layer "B.Cu") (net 3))
 (segment (start 44.858062 77.6) (end 137 77.6) (width 0.3) (layer "F.Cu") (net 6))
 (segment (start 138.2968 75.2032) (end 138.3634 75.2032) (width 0.3) (layer "F.Cu") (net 6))
 (segment (start 44.3 75.7) (end 44.3 77.041938) (width 0.3) (layer "F.Cu") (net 6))
 (segment (start 137.6 75.9) (end 138.2968 75.2032) (width 0.3) (layer "F.Cu") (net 6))
 (segment (start 44.3 75.4166) (end 44.0866 75.2032) (width 0.2) (layer "F.Cu") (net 6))
 (segment (start 137 77.6) (end 137.6 77) (width 0.3) (layer "F.Cu") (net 6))
 (segment (start 44.3 77.041938) (end 44.858062 77.6) (width 0.3) (layer "F.Cu") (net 6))
 (segment (start 44.0866 75.2032) (end 43.7 75.2032) (width 0.2) (layer "F.Cu") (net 6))
 (segment (start 138.3634 75.2032) (end 138.7 75.2032) (width 0.2) (layer "F.Cu") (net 6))
 (segment (start 137.6 77) (end 137.6 75.9) (width 0.3) (layer "F.Cu") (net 6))
 (segment (start 44.3 75.7) (end 44.3 75.4166) (width 0.2) (layer "F.Cu") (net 6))
 (segment (start 41.9032 74.7968) (end 41.3 74.7968) (width 0.2) (layer "F.Cu") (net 2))
 (segment (start 42.4 74) (end 44.6 71.8) (width 0.3) (layer "F.Cu") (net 2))
 (segment (start 133.8 71.8) (end 135.108698 73.108698) (width 0.3) (layer "F.Cu") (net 2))
 (segment (start 132.2 71.8) (end 133.8 71.8) (width 0.3) (layer "F.Cu") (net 2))
 (segment (start 135.737096 74.7968) (end 135.370148 74.429852) (width 0.2) (layer "F.Cu") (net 2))
 (segment (start 42.4 74.3) (end 41.9032 74.7968) (width 0.2) (layer "F.Cu") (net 2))
 (segment (start 135.108698 74.168402) (end 135.370148 74.429852) (width 0.3) (layer "F.Cu") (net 2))
 (segment (start 136.3 74.7968) (end 135.737096 74.7968) (width 0.2) (layer "F.Cu") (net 2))
 (segment (start 135.108698 73.108698) (end 135.108698 74.168402) (width 0.3) (layer "F.Cu") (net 2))
 (segment (start 42.4 74.3) (end 42.4 74) (width 0.3) (layer "F.Cu") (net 2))
 (segment (start 44.6 71.8) (end 132.2 71.8) (width 0.3) (layer "F.Cu") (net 2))
 (segment (start 45.2 76.825) (end 45.2 76.5) (width 0.4) (layer "F.Cu") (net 13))
 (segment (start 45.2 76.5) (end 46.7 75) (width 0.4) (layer "F.Cu") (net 13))
 (segment (start 46.7 75) (end 47.083333 75) (width 0.4) (layer "F.Cu") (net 13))
 (segment (start 116.25 75) (end 130.416667 75) (width 0.5) (layer "F.Cu") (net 7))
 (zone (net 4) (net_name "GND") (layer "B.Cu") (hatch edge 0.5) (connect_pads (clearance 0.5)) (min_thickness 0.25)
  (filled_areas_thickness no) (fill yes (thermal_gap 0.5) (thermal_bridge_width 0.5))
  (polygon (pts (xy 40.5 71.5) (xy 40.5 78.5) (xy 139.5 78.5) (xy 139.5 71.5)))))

